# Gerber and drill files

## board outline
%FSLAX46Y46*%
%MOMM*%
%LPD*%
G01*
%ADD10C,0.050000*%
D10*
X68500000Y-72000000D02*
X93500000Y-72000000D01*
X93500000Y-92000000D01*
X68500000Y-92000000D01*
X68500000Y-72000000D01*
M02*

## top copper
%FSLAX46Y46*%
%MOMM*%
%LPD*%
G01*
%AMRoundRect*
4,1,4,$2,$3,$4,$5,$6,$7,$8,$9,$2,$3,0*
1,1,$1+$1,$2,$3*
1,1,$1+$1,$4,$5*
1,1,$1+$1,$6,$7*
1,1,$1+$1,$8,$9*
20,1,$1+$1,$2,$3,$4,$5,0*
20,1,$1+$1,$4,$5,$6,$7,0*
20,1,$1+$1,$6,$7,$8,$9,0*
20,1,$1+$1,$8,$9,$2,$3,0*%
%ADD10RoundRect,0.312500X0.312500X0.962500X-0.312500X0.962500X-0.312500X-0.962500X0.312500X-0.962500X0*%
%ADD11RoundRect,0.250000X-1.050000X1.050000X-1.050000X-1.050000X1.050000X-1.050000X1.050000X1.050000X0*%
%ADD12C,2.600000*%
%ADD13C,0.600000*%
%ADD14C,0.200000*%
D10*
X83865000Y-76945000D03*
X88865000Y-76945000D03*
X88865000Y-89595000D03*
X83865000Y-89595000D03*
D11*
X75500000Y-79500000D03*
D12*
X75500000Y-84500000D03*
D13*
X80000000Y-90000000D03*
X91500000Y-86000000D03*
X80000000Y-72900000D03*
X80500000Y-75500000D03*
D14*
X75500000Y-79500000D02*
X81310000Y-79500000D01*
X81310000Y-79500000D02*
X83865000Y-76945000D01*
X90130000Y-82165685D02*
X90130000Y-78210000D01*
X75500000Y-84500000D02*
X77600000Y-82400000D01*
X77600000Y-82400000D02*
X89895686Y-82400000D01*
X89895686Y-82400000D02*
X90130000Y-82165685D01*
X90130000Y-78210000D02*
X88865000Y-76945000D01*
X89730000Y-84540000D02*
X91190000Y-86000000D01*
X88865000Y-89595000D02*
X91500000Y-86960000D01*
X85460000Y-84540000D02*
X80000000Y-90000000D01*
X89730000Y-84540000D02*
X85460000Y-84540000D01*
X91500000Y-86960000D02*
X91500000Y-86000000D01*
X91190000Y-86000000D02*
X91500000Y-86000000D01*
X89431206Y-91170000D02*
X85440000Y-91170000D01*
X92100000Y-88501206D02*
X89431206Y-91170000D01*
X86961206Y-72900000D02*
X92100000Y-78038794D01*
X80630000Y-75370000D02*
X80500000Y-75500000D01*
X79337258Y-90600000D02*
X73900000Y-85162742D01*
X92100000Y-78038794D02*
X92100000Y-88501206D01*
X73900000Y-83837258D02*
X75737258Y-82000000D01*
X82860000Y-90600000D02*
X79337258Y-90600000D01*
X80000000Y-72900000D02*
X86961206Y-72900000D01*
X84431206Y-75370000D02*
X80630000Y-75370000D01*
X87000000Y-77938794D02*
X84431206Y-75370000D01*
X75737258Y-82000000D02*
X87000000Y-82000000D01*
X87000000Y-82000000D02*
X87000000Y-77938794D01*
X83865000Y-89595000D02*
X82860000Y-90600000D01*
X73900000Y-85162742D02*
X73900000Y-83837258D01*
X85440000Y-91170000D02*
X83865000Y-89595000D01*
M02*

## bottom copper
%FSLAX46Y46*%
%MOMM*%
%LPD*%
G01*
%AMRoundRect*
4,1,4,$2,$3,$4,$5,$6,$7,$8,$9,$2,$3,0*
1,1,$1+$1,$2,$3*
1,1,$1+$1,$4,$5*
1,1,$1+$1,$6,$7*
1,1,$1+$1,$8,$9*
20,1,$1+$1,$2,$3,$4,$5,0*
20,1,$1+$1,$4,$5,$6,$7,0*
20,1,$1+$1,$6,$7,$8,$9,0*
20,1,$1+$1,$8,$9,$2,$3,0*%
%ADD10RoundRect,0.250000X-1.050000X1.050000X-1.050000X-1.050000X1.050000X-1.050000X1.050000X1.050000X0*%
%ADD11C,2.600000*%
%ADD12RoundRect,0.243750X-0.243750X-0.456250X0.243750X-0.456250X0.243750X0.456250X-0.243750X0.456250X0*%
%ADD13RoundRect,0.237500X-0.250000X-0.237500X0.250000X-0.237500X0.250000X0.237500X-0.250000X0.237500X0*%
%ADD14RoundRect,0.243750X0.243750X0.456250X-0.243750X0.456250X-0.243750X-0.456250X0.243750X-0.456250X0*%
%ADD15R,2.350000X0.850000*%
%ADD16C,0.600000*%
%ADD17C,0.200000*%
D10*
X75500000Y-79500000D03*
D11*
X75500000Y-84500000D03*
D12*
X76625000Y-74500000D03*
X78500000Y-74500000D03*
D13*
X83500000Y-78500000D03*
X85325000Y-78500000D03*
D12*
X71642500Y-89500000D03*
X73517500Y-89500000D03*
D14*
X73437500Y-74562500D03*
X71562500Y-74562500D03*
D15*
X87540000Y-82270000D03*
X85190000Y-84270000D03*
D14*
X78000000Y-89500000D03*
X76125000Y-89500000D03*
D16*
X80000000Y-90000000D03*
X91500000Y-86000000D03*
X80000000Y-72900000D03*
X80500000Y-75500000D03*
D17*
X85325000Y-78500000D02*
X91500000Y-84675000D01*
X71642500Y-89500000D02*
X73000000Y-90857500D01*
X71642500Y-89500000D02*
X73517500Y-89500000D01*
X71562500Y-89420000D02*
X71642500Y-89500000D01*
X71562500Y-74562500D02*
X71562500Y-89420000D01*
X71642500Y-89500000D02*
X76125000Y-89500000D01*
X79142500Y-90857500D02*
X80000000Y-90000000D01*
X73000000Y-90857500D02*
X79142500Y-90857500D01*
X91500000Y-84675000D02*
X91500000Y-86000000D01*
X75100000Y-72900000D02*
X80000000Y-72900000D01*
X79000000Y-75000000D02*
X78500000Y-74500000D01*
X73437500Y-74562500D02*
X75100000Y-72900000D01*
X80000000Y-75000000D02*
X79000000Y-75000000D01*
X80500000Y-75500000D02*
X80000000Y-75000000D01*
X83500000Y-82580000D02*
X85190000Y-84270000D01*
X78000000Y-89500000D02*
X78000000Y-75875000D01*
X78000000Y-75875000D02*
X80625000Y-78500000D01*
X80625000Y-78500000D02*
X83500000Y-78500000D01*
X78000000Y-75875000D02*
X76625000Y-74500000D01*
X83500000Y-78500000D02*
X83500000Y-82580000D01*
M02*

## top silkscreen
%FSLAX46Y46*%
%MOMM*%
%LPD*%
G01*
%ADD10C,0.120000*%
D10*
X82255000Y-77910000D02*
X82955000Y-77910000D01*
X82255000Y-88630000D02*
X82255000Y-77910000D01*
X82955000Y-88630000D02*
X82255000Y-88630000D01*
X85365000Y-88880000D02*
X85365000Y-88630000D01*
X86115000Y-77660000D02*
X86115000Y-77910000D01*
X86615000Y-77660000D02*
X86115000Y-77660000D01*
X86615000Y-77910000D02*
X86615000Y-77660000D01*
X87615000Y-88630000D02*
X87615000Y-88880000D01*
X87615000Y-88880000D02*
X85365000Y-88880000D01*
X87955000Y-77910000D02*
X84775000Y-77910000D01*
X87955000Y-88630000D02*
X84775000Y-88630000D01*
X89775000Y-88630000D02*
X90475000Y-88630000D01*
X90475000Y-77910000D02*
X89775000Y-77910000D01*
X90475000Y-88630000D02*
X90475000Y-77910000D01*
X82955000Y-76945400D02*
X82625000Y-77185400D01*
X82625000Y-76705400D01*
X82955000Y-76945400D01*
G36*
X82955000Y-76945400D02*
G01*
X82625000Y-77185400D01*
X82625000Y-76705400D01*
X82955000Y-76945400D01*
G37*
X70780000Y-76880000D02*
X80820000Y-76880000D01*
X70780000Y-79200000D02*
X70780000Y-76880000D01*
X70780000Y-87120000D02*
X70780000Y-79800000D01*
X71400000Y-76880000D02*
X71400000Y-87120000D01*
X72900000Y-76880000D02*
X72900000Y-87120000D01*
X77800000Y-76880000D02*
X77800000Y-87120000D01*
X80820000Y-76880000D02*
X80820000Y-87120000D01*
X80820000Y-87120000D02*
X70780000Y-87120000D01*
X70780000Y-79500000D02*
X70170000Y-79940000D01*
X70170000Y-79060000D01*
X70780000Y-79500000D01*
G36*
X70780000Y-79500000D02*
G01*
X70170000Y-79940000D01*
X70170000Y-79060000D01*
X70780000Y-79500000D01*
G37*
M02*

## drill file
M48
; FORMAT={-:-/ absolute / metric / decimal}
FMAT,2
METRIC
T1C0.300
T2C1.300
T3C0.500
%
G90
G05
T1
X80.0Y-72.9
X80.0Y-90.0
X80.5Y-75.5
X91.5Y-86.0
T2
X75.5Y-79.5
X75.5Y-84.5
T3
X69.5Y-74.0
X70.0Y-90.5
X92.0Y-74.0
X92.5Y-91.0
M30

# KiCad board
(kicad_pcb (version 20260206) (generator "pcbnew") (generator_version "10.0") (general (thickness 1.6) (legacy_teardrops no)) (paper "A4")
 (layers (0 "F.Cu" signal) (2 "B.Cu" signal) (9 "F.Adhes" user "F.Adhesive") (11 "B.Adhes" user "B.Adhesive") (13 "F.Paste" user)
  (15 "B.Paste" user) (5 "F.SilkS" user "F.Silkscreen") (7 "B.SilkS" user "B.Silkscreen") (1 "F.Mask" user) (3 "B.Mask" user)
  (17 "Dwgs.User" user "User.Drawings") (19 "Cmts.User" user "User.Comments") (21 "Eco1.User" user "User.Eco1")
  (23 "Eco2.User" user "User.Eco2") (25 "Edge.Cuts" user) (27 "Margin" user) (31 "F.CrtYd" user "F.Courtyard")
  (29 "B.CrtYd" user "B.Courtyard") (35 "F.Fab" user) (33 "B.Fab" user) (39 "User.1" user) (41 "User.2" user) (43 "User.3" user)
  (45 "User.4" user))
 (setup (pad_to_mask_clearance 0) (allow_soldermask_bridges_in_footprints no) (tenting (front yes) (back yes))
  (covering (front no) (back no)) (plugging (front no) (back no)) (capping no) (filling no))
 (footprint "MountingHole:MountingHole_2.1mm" (layer "F.Cu") (at 92.5 91)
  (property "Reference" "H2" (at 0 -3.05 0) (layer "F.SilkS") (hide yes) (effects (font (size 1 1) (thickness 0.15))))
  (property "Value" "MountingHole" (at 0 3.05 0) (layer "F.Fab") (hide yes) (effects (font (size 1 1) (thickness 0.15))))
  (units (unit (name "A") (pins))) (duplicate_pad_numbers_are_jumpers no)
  (pad "" np_thru_hole circle (at 0 0) (size 0.5 0.5) (drill 0.5) (layers "*.Cu" "*.Mask")))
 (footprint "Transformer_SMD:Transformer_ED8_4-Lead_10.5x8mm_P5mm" (layer "F.Cu") (at 86.365 83.27)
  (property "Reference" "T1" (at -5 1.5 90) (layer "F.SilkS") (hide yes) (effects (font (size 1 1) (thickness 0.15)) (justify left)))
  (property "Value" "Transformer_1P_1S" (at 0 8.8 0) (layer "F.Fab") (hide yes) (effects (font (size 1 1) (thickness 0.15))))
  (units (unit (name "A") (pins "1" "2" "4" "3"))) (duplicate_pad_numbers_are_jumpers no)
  (fp_line (start -4.11 -5.36) (end -3.41 -5.36) (stroke (width 0.12) (type default)) (layer "F.SilkS"))
  (fp_line (start -4.11 5.36) (end -4.11 -5.36) (stroke (width 0.12) (type default)) (layer "F.SilkS"))
  (fp_line (start -3.41 5.36) (end -4.11 5.36) (stroke (width 0.12) (type default)) (layer "F.SilkS"))
  (fp_line (start -1 5.61) (end -1 5.36) (stroke (width 0.12) (type default)) (layer "F.SilkS"))
  (fp_line (start -0.25 -5.61) (end -0.25 -5.36) (stroke (width 0.12) (type default)) (layer "F.SilkS"))
  (fp_line (start 0.25 -5.61) (end -0.25 -5.61) (stroke (width 0.12) (type default)) (layer "F.SilkS"))
  (fp_line (start 0.25 -5.36) (end 0.25 -5.61) (stroke (width 0.12) (type default)) (layer "F.SilkS"))
  (fp_line (start 1.25 5.36) (end 1.25 5.61) (stroke (width 0.12) (type default)) (layer "F.SilkS"))
  (fp_line (start 1.25 5.61) (end -1 5.61) (stroke (width 0.12) (type default)) (layer "F.SilkS"))
  (fp_line (start 1.59 -5.36) (end -1.59 -5.36) (stroke (width 0.12) (type default)) (layer "F.SilkS"))
  (fp_line (start 1.59 5.36) (end -1.59 5.36) (stroke (width 0.12) (type default)) (layer "F.SilkS"))
  (fp_line (start 3.41 5.36) (end 4.11 5.36) (stroke (width 0.12) (type default)) (layer "F.SilkS"))
  (fp_line (start 4.11 -5.36) (end 3.41 -5.36) (stroke (width 0.12) (type default)) (layer "F.SilkS"))
  (fp_line (start 4.11 5.36) (end 4.11 -5.36) (stroke (width 0.12) (type default)) (layer "F.SilkS"))
  (fp_poly
   (pts (xy -3.41 -6.3246) (xy -3.74 -6.0846) (xy -3.74 -6.5646) (xy -3.41 -6.3246)) (stroke (width 0.12) (type solid)) (fill yes)
   (layer "F.SilkS"))
  (pad "1" smd roundrect (at -2.5 -6.325 180) (size 1.25 2.55) (layers "F.Cu" "F.Mask" "F.Paste") (roundrect_rratio 0.25)
   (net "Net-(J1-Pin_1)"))
  (pad "2" smd roundrect (at 2.5 -6.325 180) (size 1.25 2.55) (layers "F.Cu" "F.Mask" "F.Paste") (roundrect_rratio 0.25)
   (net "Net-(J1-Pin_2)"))
  (pad "3" smd roundrect (at 2.5 6.325 180) (size 1.25 2.55) (layers "F.Cu" "F.Mask" "F.Paste") (roundrect_rratio 0.25) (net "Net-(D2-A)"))
  (pad "4" smd roundrect (at -2.5 6.325 180) (size 1.25 2.55) (layers "F.Cu" "F.Mask" "F.Paste") (roundrect_rratio 0.25) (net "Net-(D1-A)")))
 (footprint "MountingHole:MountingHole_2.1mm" (layer "F.Cu") (at 69.5 74)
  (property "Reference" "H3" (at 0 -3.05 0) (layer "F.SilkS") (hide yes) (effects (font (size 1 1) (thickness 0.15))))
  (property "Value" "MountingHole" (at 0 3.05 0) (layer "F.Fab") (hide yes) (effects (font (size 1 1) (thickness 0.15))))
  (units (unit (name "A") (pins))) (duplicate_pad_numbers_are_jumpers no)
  (pad "" np_thru_hole circle (at 0 0) (size 0.5 0.5) (drill 0.5) (layers "*.Cu" "*.Mask")))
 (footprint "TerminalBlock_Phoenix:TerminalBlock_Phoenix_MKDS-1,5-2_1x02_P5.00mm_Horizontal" (layer "F.Cu") (at 75.5 79.5 -90)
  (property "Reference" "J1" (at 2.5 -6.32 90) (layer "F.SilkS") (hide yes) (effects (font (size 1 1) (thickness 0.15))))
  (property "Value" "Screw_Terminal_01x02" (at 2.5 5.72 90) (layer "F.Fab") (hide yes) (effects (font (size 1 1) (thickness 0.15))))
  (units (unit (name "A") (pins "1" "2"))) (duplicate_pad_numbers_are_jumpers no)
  (fp_line (start -2.62 4.72) (end -2.62 -5.32) (stroke (width 0.12) (type solid)) (layer "F.SilkS"))
  (fp_line (start -0.3 4.72) (end -2.62 4.72) (stroke (width 0.12) (type solid)) (layer "F.SilkS"))
  (fp_line (start 7.62 4.72) (end 0.3 4.72) (stroke (width 0.12) (type solid)) (layer "F.SilkS"))
  (fp_line (start -2.62 4.1) (end 7.62 4.1) (stroke (width 0.12) (type solid)) (layer "F.SilkS"))
  (fp_line (start -2.62 2.6) (end 7.62 2.6) (stroke (width 0.12) (type solid)) (layer "F.SilkS"))
  (fp_line (start -2.62 -2.3) (end 7.62 -2.3) (stroke (width 0.12) (type solid)) (layer "F.SilkS"))
  (fp_line (start -2.62 -5.32) (end 7.62 -5.32) (stroke (width 0.12) (type solid)) (layer "F.SilkS"))
  (fp_line (start 7.62 -5.32) (end 7.62 4.72) (stroke (width 0.12) (type solid)) (layer "F.SilkS"))
  (fp_poly (pts (xy 0 4.72) (xy 0.44 5.33) (xy -0.44 5.33)) (stroke (width 0.12) (type solid)) (fill yes) (layer "F.SilkS"))
  (pad "1" thru_hole roundrect (at 0 0 270) (size 2.6 2.6) (drill 1.3) (layers "*.Cu" "*.Mask") (remove_unused_layers no)
   (roundrect_rratio 0.096154) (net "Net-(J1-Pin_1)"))
  (pad "2" thru_hole circle (at 5 0 270) (size 2.6 2.6) (drill 1.3) (layers "*.Cu" "*.Mask") (remove_unused_layers no)
   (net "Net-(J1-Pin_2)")))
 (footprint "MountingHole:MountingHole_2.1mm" (layer "F.Cu") (at 70 90.5)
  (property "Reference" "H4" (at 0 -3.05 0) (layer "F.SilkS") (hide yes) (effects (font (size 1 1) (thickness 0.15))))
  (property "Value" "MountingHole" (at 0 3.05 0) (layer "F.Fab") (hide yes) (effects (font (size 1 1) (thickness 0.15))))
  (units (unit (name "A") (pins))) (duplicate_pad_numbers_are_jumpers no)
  (pad "" np_thru_hole circle (at 0 0) (size 0.5 0.5) (drill 0.5) (layers "*.Cu" "*.Mask")))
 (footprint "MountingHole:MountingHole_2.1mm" (layer "F.Cu") (at 92 74)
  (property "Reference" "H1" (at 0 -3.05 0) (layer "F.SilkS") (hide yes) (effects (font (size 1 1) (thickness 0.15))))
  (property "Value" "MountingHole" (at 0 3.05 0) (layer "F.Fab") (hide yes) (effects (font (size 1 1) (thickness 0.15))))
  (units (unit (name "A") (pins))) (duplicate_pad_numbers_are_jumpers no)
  (pad "" np_thru_hole circle (at 0 0) (size 0.5 0.5) (drill 0.5) (layers "*.Cu" "*.Mask")))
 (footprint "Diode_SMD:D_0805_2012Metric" (layer "B.Cu") (at 77.5625 74.5)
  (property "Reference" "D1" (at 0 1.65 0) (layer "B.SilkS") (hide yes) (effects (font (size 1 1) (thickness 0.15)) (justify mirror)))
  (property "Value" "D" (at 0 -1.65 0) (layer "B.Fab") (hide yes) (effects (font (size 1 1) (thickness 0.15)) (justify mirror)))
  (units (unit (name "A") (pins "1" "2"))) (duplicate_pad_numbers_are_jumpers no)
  (pad "1" smd roundrect (at -0.9375 0) (size 0.975 1.4) (layers "B.Cu" "B.Mask" "B.Paste") (roundrect_rratio 0.25) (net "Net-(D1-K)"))
  (pad "2" smd roundrect (at 0.9375 0) (size 0.975 1.4) (layers "B.Cu" "B.Mask" "B.Paste") (roundrect_rratio 0.25) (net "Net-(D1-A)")))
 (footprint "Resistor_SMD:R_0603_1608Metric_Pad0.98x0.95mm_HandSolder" (layer "B.Cu") (at 84.4125 78.5)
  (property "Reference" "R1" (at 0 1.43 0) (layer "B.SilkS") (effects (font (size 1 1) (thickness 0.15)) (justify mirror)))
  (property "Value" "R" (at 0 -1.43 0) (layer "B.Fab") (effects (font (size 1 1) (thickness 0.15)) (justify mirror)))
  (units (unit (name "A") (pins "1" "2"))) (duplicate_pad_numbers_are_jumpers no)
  (pad "1" smd roundrect (at -0.9125 0) (size 0.975 0.95) (layers "B.Cu" "B.Mask" "B.Paste") (roundrect_rratio 0.25) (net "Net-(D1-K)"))
  (pad "2" smd roundrect (at 0.9125 0) (size 0.975 0.95) (layers "B.Cu" "B.Mask" "B.Paste") (roundrect_rratio 0.25) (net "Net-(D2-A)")))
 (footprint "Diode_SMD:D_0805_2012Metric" (layer "B.Cu") (at 72.58 89.5)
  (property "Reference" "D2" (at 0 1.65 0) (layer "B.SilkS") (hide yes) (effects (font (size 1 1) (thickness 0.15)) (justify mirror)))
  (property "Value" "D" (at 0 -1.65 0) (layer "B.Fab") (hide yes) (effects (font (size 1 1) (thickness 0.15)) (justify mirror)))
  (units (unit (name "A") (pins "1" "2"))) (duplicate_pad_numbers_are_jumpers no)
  (pad "1" smd roundrect (at -0.9375 0) (size 0.975 1.4) (layers "B.Cu" "B.Mask" "B.Paste") (roundrect_rratio 0.25) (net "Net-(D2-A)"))
  (pad "2" smd roundrect (at 0.9375 0) (size 0.975 1.4) (layers "B.Cu" "B.Mask" "B.Paste") (roundrect_rratio 0.25) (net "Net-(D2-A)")))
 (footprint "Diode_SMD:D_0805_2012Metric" (layer "B.Cu") (at 72.5 74.5625 180)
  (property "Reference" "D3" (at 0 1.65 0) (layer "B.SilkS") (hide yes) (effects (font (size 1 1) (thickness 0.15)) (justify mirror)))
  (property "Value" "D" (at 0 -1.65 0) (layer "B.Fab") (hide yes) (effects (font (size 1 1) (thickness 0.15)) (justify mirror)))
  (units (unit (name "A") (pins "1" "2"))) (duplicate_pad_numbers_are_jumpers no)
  (pad "1" smd roundrect (at -0.9375 0 180) (size 0.975 1.4) (layers "B.Cu" "B.Mask" "B.Paste") (roundrect_rratio 0.25) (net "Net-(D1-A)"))
  (pad "2" smd roundrect (at 0.9375 0 180) (size 0.975 1.4) (layers "B.Cu" "B.Mask" "B.Paste") (roundrect_rratio 0.25) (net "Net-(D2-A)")))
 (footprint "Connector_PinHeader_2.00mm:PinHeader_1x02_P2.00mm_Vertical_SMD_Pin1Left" (layer "B.Cu") (at 86.365 83.27 180)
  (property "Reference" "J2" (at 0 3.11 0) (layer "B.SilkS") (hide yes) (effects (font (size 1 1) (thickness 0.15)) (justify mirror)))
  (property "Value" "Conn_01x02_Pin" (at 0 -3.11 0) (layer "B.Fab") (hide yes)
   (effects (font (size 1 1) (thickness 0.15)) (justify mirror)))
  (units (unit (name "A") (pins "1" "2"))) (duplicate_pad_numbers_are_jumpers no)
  (pad "1" smd rect (at -1.175 1 180) (size 2.35 0.85) (layers "B.Cu" "B.Mask" "B.Paste") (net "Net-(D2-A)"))
  (pad "2" smd rect (at 1.175 -1 180) (size 2.35 0.85) (layers "B.Cu" "B.Mask" "B.Paste") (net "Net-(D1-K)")))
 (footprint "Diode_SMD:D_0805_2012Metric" (layer "B.Cu") (at 77.0625 89.5 180)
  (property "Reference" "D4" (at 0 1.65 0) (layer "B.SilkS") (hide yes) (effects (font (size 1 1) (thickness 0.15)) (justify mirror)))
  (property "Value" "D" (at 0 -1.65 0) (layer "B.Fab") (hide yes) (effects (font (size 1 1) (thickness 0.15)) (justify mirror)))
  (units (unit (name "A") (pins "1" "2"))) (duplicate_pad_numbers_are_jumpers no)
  (pad "1" smd roundrect (at -0.9375 0 180) (size 0.975 1.4) (layers "B.Cu" "B.Mask" "B.Paste") (roundrect_rratio 0.25) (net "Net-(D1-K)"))
  (pad "2" smd roundrect (at 0.9375 0 180) (size 0.975 1.4) (layers "B.Cu" "B.Mask" "B.Paste") (roundrect_rratio 0.25) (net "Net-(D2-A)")))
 (gr_rect (start 68.5 72) (end 93.5 92) (stroke (width 0.05) (type default)) (fill no) (layer "Edge.Cuts"))
 (segment (start 75.5 79.5) (end 81.31 79.5) (width 0.2) (layer "F.Cu") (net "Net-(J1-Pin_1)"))
 (segment (start 81.31 79.5) (end 83.865 76.945) (width 0.2) (layer "F.Cu") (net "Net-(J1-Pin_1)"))
 (segment (start 90.13 82.165685) (end 90.13 78.21) (width 0.2) (layer "F.Cu") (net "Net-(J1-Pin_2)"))
 (segment (start 75.5 84.5) (end 77.6 82.4) (width 0.2) (layer "F.Cu") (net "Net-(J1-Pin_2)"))
 (segment (start 77.6 82.4) (end 89.895686 82.4) (width 0.2) (layer "F.Cu") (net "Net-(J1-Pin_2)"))
 (segment (start 89.895686 82.4) (end 90.13 82.165685) (width 0.2) (layer "F.Cu") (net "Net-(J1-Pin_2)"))
 (segment (start 90.13 78.21) (end 88.865 76.945) (width 0.2) (layer "F.Cu") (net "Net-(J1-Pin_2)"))
 (segment (start 89.73 84.54) (end 91.19 86) (width 0.2) (layer "F.Cu") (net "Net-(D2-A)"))
 (segment (start 88.865 89.595) (end 91.5 86.96) (width 0.2) (layer "F.Cu") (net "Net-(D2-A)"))
 (segment (start 85.46 84.54) (end 80 90) (width 0.2) (layer "F.Cu") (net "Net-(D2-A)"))
 (segment (start 89.73 84.54) (end 85.46 84.54) (width 0.2) (layer "F.Cu") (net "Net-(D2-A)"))
 (segment (start 91.5 86.96) (end 91.5 86) (width 0.2) (layer "F.Cu") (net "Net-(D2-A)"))
 (segment (start 91.19 86) (end 91.5 86) (width 0.2) (layer "F.Cu") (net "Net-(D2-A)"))
 (via (at 80 90) (size 0.6) (drill 0.3) (layers "F.Cu" "B.Cu") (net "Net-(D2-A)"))
 (via (at 91.5 86) (size 0.6) (drill 0.3) (layers "F.Cu" "B.Cu") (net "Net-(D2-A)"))
 (segment (start 85.325 78.5) (end 91.5 84.675) (width 0.2) (layer "B.Cu") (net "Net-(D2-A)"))
 (segment (start 71.6425 89.5) (end 73 90.8575) (width 0.2) (layer "B.Cu") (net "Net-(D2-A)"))
 (segment (start 71.6425 89.5) (end 73.5175 89.5) (width 0.2) (layer "B.Cu") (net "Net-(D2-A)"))
 (segment (start 71.5625 89.42) (end 71.6425 89.5) (width 0.2) (layer "B.Cu") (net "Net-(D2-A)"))
 (segment (start 71.5625 74.5625) (end 71.5625 89.42) (width 0.2) (layer "B.Cu") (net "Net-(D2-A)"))
 (segment (start 71.6425 89.5) (end 76.125 89.5) (width 0.2) (layer "B.Cu") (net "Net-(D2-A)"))
 (segment (start 79.1425 90.8575) (end 80 90) (width 0.2) (layer "B.Cu") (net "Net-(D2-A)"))
 (segment (start 73 90.8575) (end 79.1425 90.8575) (width 0.2) (layer "B.Cu") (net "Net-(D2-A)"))
 (segment (start 91.5 84.675) (end 91.5 86) (width 0.2) (layer "B.Cu") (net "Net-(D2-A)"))
 (segment (start 89.431206 91.17) (end 85.44 91.17) (width 0.2) (layer "F.Cu") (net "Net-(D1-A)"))
 (segment (start 92.1 88.501206) (end 89.431206 91.17) (width 0.2) (layer "F.Cu") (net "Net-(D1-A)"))
 (segment (start 86.961206 72.9) (end 92.1 78.038794) (width 0.2) (layer "F.Cu") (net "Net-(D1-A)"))
 (segment (start 80.63 75.37) (end 80.5 75.5) (width 0.2) (layer "F.Cu") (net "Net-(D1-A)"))
 (segment (start 79.337258 90.6) (end 73.9 85.162742) (width 0.2) (layer "F.Cu") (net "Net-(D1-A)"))
 (segment (start 92.1 78.038794) (end 92.1 88.501206) (width 0.2) (layer "F.Cu") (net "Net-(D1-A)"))
 (segment (start 73.9 83.837258) (end 75.737258 82) (width 0.2) (layer "F.Cu") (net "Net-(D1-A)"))
 (segment (start 82.86 90.6) (end 79.337258 90.6) (width 0.2) (layer "F.Cu") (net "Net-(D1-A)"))
 (segment (start 80 72.9) (end 86.961206 72.9) (width 0.2) (layer "F.Cu") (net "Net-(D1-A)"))
 (segment (start 84.431206 75.37) (end 80.63 75.37) (width 0.2) (layer "F.Cu") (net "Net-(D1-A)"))
 (segment (start 87 77.938794) (end 84.431206 75.37) (width 0.2) (layer "F.Cu") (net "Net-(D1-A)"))
 (segment (start 75.737258 82) (end 87 82) (width 0.2) (layer "F.Cu") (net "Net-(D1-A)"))
 (segment (start 87 82) (end 87 77.938794) (width 0.2) (layer "F.Cu") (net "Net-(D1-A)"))
 (segment (start 83.865 89.595) (end 82.86 90.6) (width 0.2) (layer "F.Cu") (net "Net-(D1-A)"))
 (segment (start 73.9 85.162742) (end 73.9 83.837258) (width 0.2) (layer "F.Cu") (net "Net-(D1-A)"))
 (segment (start 85.44 91.17) (end 83.865 89.595) (width 0.2) (layer "F.Cu") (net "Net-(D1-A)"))
 (via (at 80 72.9) (size 0.6) (drill 0.3) (layers "F.Cu" "B.Cu") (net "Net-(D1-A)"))
 (via (at 80.5 75.5) (size 0.6) (drill 0.3) (layers "F.Cu" "B.Cu") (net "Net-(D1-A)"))
 (segment (start 75.1 72.9) (end 80 72.9) (width 0.2) (layer "B.Cu") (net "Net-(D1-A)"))
 (segment (start 79 75) (end 78.5 74.5) (width 0.2) (layer "B.Cu") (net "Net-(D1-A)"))
 (segment (start 73.4375 74.5625) (end 75.1 72.9) (width 0.2) (layer "B.Cu") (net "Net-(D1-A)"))
 (segment (start 80 75) (end 79 75) (width 0.2) (layer "B.Cu") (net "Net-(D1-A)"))
 (segment (start 80.5 75.5) (end 80 75) (width 0.2) (layer "B.Cu") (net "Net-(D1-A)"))
 (segment (start 83.5 82.58) (end 85.19 84.27) (width 0.2) (layer "B.Cu") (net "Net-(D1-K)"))
 (segment (start 78 89.5) (end 78 75.875) (width 0.2) (layer "B.Cu") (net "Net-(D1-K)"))
 (segment (start 78 75.875) (end 80.625 78.5) (width 0.2) (layer "B.Cu") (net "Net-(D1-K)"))
 (segment (start 80.625 78.5) (end 83.5 78.5) (width 0.2) (layer "B.Cu") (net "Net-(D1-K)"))
 (segment (start 78 75.875) (end 76.625 74.5) (width 0.2) (layer "B.Cu") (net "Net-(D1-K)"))
 (segment (start 83.5 78.5) (end 83.5 82.58) (width 0.2) (layer "B.Cu") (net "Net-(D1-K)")))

